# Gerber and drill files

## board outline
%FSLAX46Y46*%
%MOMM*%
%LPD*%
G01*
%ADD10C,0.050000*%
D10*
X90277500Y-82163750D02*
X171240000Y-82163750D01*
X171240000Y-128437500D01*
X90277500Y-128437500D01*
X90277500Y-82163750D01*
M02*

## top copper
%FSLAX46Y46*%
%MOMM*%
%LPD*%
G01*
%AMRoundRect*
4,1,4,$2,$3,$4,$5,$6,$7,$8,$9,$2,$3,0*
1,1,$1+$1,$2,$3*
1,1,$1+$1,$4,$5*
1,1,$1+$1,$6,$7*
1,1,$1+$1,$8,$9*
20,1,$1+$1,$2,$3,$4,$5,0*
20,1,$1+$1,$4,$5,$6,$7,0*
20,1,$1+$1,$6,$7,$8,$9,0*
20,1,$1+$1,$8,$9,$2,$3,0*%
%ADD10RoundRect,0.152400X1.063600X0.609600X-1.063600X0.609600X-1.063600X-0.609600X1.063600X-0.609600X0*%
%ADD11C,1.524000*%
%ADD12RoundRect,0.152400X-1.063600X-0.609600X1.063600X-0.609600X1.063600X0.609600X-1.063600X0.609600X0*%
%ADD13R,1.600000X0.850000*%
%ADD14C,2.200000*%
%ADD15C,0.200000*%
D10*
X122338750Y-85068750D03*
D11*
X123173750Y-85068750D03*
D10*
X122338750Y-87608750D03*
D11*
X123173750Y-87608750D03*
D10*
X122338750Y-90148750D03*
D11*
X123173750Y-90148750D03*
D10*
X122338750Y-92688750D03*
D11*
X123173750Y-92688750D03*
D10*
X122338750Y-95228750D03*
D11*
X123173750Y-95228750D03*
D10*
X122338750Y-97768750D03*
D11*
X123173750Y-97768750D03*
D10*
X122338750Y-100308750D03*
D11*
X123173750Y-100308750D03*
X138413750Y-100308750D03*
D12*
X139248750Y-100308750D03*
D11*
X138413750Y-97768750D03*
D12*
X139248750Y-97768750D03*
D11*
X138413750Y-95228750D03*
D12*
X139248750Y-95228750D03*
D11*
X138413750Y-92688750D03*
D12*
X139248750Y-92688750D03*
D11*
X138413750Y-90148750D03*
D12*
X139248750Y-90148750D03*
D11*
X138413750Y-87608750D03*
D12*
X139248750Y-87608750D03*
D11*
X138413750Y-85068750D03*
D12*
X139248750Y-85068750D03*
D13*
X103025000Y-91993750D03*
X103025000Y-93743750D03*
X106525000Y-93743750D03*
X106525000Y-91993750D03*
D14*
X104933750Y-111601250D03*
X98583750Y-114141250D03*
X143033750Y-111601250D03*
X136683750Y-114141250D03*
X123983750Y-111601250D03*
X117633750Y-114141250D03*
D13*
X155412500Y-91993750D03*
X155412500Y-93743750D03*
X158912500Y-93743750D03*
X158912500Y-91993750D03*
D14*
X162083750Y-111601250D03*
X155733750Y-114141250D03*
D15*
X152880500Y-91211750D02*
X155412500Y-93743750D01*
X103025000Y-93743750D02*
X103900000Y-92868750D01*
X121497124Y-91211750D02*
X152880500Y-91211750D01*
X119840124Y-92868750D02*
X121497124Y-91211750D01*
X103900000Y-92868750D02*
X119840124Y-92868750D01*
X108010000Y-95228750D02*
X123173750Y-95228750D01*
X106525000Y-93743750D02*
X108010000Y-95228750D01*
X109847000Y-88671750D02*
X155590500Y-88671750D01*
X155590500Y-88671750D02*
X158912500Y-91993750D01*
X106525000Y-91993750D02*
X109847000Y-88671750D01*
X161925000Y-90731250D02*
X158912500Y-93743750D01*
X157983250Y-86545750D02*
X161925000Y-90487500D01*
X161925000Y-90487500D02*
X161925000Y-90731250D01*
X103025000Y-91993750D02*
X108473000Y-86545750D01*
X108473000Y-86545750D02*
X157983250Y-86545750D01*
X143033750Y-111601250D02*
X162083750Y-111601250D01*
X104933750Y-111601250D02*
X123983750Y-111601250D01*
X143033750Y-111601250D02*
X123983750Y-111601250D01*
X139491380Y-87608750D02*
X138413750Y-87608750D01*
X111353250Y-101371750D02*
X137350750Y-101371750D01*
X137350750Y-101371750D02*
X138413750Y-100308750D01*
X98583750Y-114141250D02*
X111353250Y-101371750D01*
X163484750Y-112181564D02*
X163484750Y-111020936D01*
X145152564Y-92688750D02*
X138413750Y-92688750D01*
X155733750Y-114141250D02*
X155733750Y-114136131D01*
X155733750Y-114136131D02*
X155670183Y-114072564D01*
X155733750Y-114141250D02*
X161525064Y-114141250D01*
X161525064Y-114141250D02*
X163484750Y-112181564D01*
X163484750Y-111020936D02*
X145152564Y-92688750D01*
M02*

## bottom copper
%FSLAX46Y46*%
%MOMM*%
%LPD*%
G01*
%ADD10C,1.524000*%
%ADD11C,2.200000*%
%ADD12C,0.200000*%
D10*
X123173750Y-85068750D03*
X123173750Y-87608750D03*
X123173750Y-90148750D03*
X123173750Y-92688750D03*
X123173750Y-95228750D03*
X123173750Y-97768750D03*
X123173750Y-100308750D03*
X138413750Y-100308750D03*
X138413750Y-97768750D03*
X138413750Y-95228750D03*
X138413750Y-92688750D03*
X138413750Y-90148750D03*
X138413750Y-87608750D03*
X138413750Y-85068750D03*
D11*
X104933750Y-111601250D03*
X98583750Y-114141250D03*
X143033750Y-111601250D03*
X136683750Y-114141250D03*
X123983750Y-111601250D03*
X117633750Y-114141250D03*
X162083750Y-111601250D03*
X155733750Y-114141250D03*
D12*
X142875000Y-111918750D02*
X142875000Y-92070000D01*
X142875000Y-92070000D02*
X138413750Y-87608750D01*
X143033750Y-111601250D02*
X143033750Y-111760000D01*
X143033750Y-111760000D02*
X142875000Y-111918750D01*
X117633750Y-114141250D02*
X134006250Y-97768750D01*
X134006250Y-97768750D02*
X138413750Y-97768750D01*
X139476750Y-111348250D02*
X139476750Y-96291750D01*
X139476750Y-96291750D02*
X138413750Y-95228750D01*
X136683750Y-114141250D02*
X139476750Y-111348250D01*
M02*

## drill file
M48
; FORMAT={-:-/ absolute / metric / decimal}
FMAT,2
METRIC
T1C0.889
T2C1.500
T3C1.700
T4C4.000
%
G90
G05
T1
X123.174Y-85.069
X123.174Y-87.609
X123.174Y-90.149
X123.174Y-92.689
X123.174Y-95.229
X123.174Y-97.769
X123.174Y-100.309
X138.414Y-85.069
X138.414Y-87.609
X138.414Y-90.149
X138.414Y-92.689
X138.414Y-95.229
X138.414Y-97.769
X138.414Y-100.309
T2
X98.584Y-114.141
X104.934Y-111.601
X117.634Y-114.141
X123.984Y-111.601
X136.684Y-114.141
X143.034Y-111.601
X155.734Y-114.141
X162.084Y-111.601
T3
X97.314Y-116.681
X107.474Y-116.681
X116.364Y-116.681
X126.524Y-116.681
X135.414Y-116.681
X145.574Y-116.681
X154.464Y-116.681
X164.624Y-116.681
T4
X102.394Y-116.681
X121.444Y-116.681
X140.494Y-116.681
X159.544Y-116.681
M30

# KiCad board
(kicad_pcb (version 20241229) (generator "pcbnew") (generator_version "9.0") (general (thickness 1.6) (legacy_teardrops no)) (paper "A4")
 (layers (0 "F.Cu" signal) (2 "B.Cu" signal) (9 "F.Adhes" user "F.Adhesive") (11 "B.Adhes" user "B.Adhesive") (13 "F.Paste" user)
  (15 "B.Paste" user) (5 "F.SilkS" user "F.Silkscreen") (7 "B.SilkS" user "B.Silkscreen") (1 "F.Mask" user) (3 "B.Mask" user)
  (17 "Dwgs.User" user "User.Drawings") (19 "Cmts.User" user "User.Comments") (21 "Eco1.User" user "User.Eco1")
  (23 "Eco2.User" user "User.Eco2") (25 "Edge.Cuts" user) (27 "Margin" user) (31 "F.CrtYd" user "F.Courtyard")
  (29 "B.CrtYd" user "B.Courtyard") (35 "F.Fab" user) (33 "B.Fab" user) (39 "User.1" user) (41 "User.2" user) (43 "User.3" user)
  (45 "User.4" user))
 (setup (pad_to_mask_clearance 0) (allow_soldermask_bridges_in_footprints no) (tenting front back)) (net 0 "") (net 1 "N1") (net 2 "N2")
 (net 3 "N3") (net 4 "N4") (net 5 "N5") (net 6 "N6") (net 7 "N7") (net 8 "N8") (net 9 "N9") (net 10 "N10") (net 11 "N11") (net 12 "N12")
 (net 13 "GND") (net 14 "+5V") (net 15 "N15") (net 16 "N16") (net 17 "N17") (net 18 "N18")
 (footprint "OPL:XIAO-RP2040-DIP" (layer "F.Cu") (at 130.79375 92.68875)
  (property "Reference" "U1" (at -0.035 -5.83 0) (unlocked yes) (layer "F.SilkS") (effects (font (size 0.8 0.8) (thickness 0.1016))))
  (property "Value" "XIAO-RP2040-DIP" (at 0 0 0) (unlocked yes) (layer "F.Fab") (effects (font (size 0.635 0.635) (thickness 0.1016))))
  (pad "1" smd roundrect (at -8.455 -7.62 180) (size 2.432 1.524) (layers "F.Cu" "F.Mask") (roundrect_rratio 0.1) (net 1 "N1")
   (thermal_bridge_angle 45))
  (pad "1" thru_hole circle (at -7.62 -7.62 180) (size 1.524 1.524) (drill 0.889) (layers "*.Cu" "*.Mask") (remove_unused_layers no)
   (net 1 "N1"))
  (pad "2" smd roundrect (at -8.455 -5.08 180) (size 2.432 1.524) (layers "F.Cu" "F.Mask") (roundrect_rratio 0.1) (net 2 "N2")
   (thermal_bridge_angle 45))
  (pad "2" thru_hole circle (at -7.62 -5.08 180) (size 1.524 1.524) (drill 0.889) (layers "*.Cu" "*.Mask") (remove_unused_layers no)
   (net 2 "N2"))
  (pad "3" smd roundrect (at -8.455 -2.54 180) (size 2.432 1.524) (layers "F.Cu" "F.Mask") (roundrect_rratio 0.1) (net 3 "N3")
   (thermal_bridge_angle 45))
  (pad "3" thru_hole circle (at -7.62 -2.54 180) (size 1.524 1.524) (drill 0.889) (layers "*.Cu" "*.Mask") (remove_unused_layers no)
   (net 3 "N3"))
  (pad "4" smd roundrect (at -8.455 0 180) (size 2.432 1.524) (layers "F.Cu" "F.Mask") (roundrect_rratio 0.1) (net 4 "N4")
   (thermal_bridge_angle 45))
  (pad "4" thru_hole circle (at -7.62 0 180) (size 1.524 1.524) (drill 0.889) (layers "*.Cu" "*.Mask") (remove_unused_layers no)
   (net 4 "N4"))
  (pad "5" smd roundrect (at -8.455 2.54 180) (size 2.432 1.524) (layers "F.Cu" "F.Mask") (roundrect_rratio 0.1) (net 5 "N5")
   (thermal_bridge_angle 45))
  (pad "5" thru_hole circle (at -7.62 2.54 180) (size 1.524 1.524) (drill 0.889) (layers "*.Cu" "*.Mask") (remove_unused_layers no)
   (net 5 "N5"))
  (pad "6" smd roundrect (at -8.455 5.08 180) (size 2.432 1.524) (layers "F.Cu" "F.Mask") (roundrect_rratio 0.1) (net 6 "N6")
   (thermal_bridge_angle 45))
  (pad "6" thru_hole circle (at -7.62 5.08 180) (size 1.524 1.524) (drill 0.889) (layers "*.Cu" "*.Mask") (remove_unused_layers no)
   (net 6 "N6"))
  (pad "7" smd roundrect (at -8.455 7.62 180) (size 2.432 1.524) (layers "F.Cu" "F.Mask") (roundrect_rratio 0.1) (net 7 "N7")
   (thermal_bridge_angle 45))
  (pad "7" thru_hole circle (at -7.62 7.62 180) (size 1.524 1.524) (drill 0.889) (layers "*.Cu" "*.Mask") (remove_unused_layers no)
   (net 7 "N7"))
  (pad "8" thru_hole circle (at 7.62 7.62) (size 1.524 1.524) (drill 0.889) (layers "*.Cu" "*.Mask") (remove_unused_layers no) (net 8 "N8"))
  (pad "8" smd roundrect (at 8.455 7.62) (size 2.432 1.524) (layers "F.Cu" "F.Mask") (roundrect_rratio 0.1) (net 8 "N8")
   (thermal_bridge_angle 45))
  (pad "9" thru_hole circle (at 7.62 5.08) (size 1.524 1.524) (drill 0.889) (layers "*.Cu" "*.Mask") (remove_unused_layers no) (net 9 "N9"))
  (pad "9" smd roundrect (at 8.455 5.08) (size 2.432 1.524) (layers "F.Cu" "F.Mask") (roundrect_rratio 0.1) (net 9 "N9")
   (thermal_bridge_angle 45))
  (pad "10" thru_hole circle (at 7.62 2.54) (size 1.524 1.524) (drill 0.889) (layers "*.Cu" "*.Mask") (remove_unused_layers no)
   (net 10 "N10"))
  (pad "10" smd roundrect (at 8.455 2.54) (size 2.432 1.524) (layers "F.Cu" "F.Mask") (roundrect_rratio 0.1) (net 10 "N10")
   (thermal_bridge_angle 45))
  (pad "11" thru_hole circle (at 7.62 0) (size 1.524 1.524) (drill 0.889) (layers "*.Cu" "*.Mask") (remove_unused_layers no) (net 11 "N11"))
  (pad "11" smd roundrect (at 8.455 0) (size 2.432 1.524) (layers "F.Cu" "F.Mask") (roundrect_rratio 0.1) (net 11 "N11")
   (thermal_bridge_angle 45))
  (pad "12" thru_hole circle (at 7.62 -2.54) (size 1.524 1.524) (drill 0.889) (layers "*.Cu" "*.Mask") (remove_unused_layers no)
   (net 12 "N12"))
  (pad "12" smd roundrect (at 8.455 -2.54) (size 2.432 1.524) (layers "F.Cu" "F.Mask") (roundrect_rratio 0.1) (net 12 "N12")
   (thermal_bridge_angle 45))
  (pad "13" thru_hole circle (at 7.62 -5.08) (size 1.524 1.524) (drill 0.889) (layers "*.Cu" "*.Mask") (remove_unused_layers no)
   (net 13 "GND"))
  (pad "13" smd roundrect (at 8.455 -5.08) (size 2.432 1.524) (layers "F.Cu" "F.Mask") (roundrect_rratio 0.1) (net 13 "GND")
   (thermal_bridge_angle 45))
  (pad "14" thru_hole circle (at 7.62 -7.62) (size 1.524 1.524) (drill 0.889) (layers "*.Cu" "*.Mask") (remove_unused_layers no)
   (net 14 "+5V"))
  (pad "14" smd roundrect (at 8.455 -7.62) (size 2.432 1.524) (layers "F.Cu" "F.Mask") (roundrect_rratio 0.1) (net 14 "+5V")
   (thermal_bridge_angle 45)))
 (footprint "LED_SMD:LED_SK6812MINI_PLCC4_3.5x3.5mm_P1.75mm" (layer "F.Cu") (at 104.775 92.86875)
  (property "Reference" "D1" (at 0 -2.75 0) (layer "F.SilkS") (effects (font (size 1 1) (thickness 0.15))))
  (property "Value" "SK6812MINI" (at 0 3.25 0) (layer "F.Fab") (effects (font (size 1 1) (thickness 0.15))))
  (pad "1" smd rect (at -1.75 -0.875) (size 1.6 0.85) (layers "F.Cu" "F.Mask" "F.Paste") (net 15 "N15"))
  (pad "2" smd rect (at -1.75 0.875) (size 1.6 0.85) (layers "F.Cu" "F.Mask" "F.Paste") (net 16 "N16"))
  (pad "3" smd rect (at 1.75 0.875) (size 1.6 0.85) (layers "F.Cu" "F.Mask" "F.Paste") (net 5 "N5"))
  (pad "4" smd rect (at 1.75 -0.875) (size 1.6 0.85) (layers "F.Cu" "F.Mask" "F.Paste") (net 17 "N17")))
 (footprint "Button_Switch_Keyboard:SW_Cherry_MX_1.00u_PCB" (layer "F.Cu") (at 104.93375 111.60125)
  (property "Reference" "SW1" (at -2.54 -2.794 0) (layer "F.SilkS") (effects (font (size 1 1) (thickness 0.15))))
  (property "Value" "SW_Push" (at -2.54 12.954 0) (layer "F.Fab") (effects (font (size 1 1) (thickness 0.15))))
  (pad "" np_thru_hole circle (at -7.62 5.08) (size 1.7 1.7) (drill 1.7) (layers "*.Cu" "*.Mask"))
  (pad "" np_thru_hole circle (at -2.54 5.08) (size 4 4) (drill 4) (layers "*.Cu" "*.Mask"))
  (pad "" np_thru_hole circle (at 2.54 5.08) (size 1.7 1.7) (drill 1.7) (layers "*.Cu" "*.Mask"))
  (pad "1" thru_hole circle (at 0 0) (size 2.2 2.2) (drill 1.5) (layers "*.Cu" "*.Mask") (remove_unused_layers no) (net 13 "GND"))
  (pad "2" thru_hole circle (at -6.35 2.54) (size 2.2 2.2) (drill 1.5) (layers "*.Cu" "*.Mask") (remove_unused_layers no) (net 8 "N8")))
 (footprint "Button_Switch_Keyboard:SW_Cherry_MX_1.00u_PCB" (layer "F.Cu") (at 143.03375 111.60125)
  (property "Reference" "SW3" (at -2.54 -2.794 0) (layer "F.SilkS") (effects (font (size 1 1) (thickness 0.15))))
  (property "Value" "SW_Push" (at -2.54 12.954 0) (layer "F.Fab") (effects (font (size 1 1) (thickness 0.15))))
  (pad "" np_thru_hole circle (at -7.62 5.08) (size 1.7 1.7) (drill 1.7) (layers "*.Cu" "*.Mask"))
  (pad "" np_thru_hole circle (at -2.54 5.08) (size 4 4) (drill 4) (layers "*.Cu" "*.Mask"))
  (pad "" np_thru_hole circle (at 2.54 5.08) (size 1.7 1.7) (drill 1.7) (layers "*.Cu" "*.Mask"))
  (pad "1" thru_hole circle (at 0 0) (size 2.2 2.2) (drill 1.5) (layers "*.Cu" "*.Mask") (remove_unused_layers no) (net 13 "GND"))
  (pad "2" thru_hole circle (at -6.35 2.54) (size 2.2 2.2) (drill 1.5) (layers "*.Cu" "*.Mask") (remove_unused_layers no) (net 10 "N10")))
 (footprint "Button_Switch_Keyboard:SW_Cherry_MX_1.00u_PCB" (layer "F.Cu") (at 123.98375 111.60125)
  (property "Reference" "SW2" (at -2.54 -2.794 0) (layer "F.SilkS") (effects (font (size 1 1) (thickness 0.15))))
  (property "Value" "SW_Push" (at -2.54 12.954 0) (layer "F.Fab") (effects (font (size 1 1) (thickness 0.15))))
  (pad "" np_thru_hole circle (at -7.62 5.08) (size 1.7 1.7) (drill 1.7) (layers "*.Cu" "*.Mask"))
  (pad "" np_thru_hole circle (at -2.54 5.08) (size 4 4) (drill 4) (layers "*.Cu" "*.Mask"))
  (pad "" np_thru_hole circle (at 2.54 5.08) (size 1.7 1.7) (drill 1.7) (layers "*.Cu" "*.Mask"))
  (pad "1" thru_hole circle (at 0 0) (size 2.2 2.2) (drill 1.5) (layers "*.Cu" "*.Mask") (remove_unused_layers no) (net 13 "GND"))
  (pad "2" thru_hole circle (at -6.35 2.54) (size 2.2 2.2) (drill 1.5) (layers "*.Cu" "*.Mask") (remove_unused_layers no) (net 9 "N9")))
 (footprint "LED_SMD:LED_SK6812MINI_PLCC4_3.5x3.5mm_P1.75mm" (layer "F.Cu") (at 157.1625 92.86875)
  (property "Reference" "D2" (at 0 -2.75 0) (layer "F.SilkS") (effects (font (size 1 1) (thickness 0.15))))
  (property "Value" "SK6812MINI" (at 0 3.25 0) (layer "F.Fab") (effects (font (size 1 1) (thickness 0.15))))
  (pad "1" smd rect (at -1.75 -0.875) (size 1.6 0.85) (layers "F.Cu" "F.Mask" "F.Paste") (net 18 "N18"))
  (pad "2" smd rect (at -1.75 0.875) (size 1.6 0.85) (layers "F.Cu" "F.Mask" "F.Paste") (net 16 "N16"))
  (pad "3" smd rect (at 1.75 0.875) (size 1.6 0.85) (layers "F.Cu" "F.Mask" "F.Paste") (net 15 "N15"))
  (pad "4" smd rect (at 1.75 -0.875) (size 1.6 0.85) (layers "F.Cu" "F.Mask" "F.Paste") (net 17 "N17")))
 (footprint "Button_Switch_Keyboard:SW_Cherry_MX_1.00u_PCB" (layer "F.Cu") (at 162.08375 111.60125)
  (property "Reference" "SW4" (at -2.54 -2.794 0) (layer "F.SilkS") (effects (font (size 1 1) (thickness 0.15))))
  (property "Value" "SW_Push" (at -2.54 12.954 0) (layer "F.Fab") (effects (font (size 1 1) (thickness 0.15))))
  (pad "" np_thru_hole circle (at -7.62 5.08) (size 1.7 1.7) (drill 1.7) (layers "*.Cu" "*.Mask"))
  (pad "" np_thru_hole circle (at -2.54 5.08) (size 4 4) (drill 4) (layers "*.Cu" "*.Mask"))
  (pad "" np_thru_hole circle (at 2.54 5.08) (size 1.7 1.7) (drill 1.7) (layers "*.Cu" "*.Mask"))
  (pad "1" thru_hole circle (at 0 0) (size 2.2 2.2) (drill 1.5) (layers "*.Cu" "*.Mask") (remove_unused_layers no) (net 13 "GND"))
  (pad "2" thru_hole circle (at -6.35 2.54) (size 2.2 2.2) (drill 1.5) (layers "*.Cu" "*.Mask") (remove_unused_layers no) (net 11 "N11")))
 (gr_rect (start 90.2775 82.16375) (end 171.24 128.4375) (stroke (width 0.05) (type solid)) (fill no) (layer "Edge.Cuts"))
 (segment (start 152.8805 91.21175) (end 155.4125 93.74375) (width 0.2) (layer "F.Cu") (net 16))
 (segment (start 103.025 93.74375) (end 103.9 92.86875) (width 0.2) (layer "F.Cu") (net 16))
 (segment (start 121.497124 91.21175) (end 152.8805 91.21175) (width 0.2) (layer "F.Cu") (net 16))
 (segment (start 119.840124 92.86875) (end 121.497124 91.21175) (width 0.2) (layer "F.Cu") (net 16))
 (segment (start 103.9 92.86875) (end 119.840124 92.86875) (width 0.2) (layer "F.Cu") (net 16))
 (segment (start 108.01 95.22875) (end 123.17375 95.22875) (width 0.2) (layer "F.Cu") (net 5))
 (segment (start 106.525 93.74375) (end 108.01 95.22875) (width 0.2) (layer "F.Cu") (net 5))
 (segment (start 109.847 88.67175) (end 155.5905 88.67175) (width 0.2) (layer "F.Cu") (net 17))
 (segment (start 155.5905 88.67175) (end 158.9125 91.99375) (width 0.2) (layer "F.Cu") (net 17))
 (segment (start 106.525 91.99375) (end 109.847 88.67175) (width 0.2) (layer "F.Cu") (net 17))
 (segment (start 161.925 90.73125) (end 158.9125 93.74375) (width 0.2) (layer "F.Cu") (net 15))
 (segment (start 157.98325 86.54575) (end 161.925 90.4875) (width 0.2) (layer "F.Cu") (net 15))
 (segment (start 161.925 90.4875) (end 161.925 90.73125) (width 0.2) (layer "F.Cu") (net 15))
 (segment (start 103.025 91.99375) (end 108.473 86.54575) (width 0.2) (layer "F.Cu") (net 15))
 (segment (start 108.473 86.54575) (end 157.98325 86.54575) (width 0.2) (layer "F.Cu") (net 15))
 (segment (start 143.03375 111.60125) (end 162.08375 111.60125) (width 0.2) (layer "F.Cu") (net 13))
 (segment (start 104.93375 111.60125) (end 123.98375 111.60125) (width 0.2) (layer "F.Cu") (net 13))
 (segment (start 143.03375 111.60125) (end 123.98375 111.60125) (width 0.2) (layer "F.Cu") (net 13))
 (segment (start 139.49138 87.60875) (end 138.41375 87.60875) (width 0.2) (layer "F.Cu") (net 13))
 (segment (start 142.875 111.91875) (end 142.875 92.07) (width 0.2) (layer "B.Cu") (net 13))
 (segment (start 142.875 92.07) (end 138.41375 87.60875) (width 0.2) (layer "B.Cu") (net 13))
 (segment (start 143.03375 111.60125) (end 143.03375 111.76) (width 0.2) (layer "B.Cu") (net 13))
 (segment (start 143.03375 111.76) (end 142.875 111.91875) (width 0.2) (layer "B.Cu") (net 13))
 (segment (start 111.35325 101.37175) (end 137.35075 101.37175) (width 0.2) (layer "F.Cu") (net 8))
 (segment (start 137.35075 101.37175) (end 138.41375 100.30875) (width 0.2) (layer "F.Cu") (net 8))
 (segment (start 98.58375 114.14125) (end 111.35325 101.37175) (width 0.2) (layer "F.Cu") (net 8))
 (segment (start 117.63375 114.14125) (end 134.00625 97.76875) (width 0.2) (layer "B.Cu") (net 9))
 (segment (start 134.00625 97.76875) (end 138.41375 97.76875) (width 0.2) (layer "B.Cu") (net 9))
 (segment (start 139.47675 111.34825) (end 139.47675 96.29175) (width 0.2) (layer "B.Cu") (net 10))
 (segment (start 139.47675 96.29175) (end 138.41375 95.22875) (width 0.2) (layer "B.Cu") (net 10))
 (segment (start 136.68375 114.14125) (end 139.47675 111.34825) (width 0.2) (layer "B.Cu") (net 10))
 (segment (start 163.48475 112.181564) (end 163.48475 111.020936) (width 0.2) (layer "F.Cu") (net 11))
 (segment (start 145.152564 92.68875) (end 138.41375 92.68875) (width 0.2) (layer "F.Cu") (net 11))
 (segment (start 155.73375 114.14125) (end 155.73375 114.136131) (width 0.2) (layer "F.Cu") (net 11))
 (segment (start 155.73375 114.136131) (end 155.670183 114.072564) (width 0.2) (layer "F.Cu") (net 11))
 (segment (start 155.73375 114.14125) (end 161.525064 114.14125) (width 0.2) (layer "F.Cu") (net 11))
 (segment (start 161.525064 114.14125) (end 163.48475 112.181564) (width 0.2) (layer "F.Cu") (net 11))
 (segment (start 163.48475 111.020936) (end 145.152564 92.68875) (width 0.2) (layer "F.Cu") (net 11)))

